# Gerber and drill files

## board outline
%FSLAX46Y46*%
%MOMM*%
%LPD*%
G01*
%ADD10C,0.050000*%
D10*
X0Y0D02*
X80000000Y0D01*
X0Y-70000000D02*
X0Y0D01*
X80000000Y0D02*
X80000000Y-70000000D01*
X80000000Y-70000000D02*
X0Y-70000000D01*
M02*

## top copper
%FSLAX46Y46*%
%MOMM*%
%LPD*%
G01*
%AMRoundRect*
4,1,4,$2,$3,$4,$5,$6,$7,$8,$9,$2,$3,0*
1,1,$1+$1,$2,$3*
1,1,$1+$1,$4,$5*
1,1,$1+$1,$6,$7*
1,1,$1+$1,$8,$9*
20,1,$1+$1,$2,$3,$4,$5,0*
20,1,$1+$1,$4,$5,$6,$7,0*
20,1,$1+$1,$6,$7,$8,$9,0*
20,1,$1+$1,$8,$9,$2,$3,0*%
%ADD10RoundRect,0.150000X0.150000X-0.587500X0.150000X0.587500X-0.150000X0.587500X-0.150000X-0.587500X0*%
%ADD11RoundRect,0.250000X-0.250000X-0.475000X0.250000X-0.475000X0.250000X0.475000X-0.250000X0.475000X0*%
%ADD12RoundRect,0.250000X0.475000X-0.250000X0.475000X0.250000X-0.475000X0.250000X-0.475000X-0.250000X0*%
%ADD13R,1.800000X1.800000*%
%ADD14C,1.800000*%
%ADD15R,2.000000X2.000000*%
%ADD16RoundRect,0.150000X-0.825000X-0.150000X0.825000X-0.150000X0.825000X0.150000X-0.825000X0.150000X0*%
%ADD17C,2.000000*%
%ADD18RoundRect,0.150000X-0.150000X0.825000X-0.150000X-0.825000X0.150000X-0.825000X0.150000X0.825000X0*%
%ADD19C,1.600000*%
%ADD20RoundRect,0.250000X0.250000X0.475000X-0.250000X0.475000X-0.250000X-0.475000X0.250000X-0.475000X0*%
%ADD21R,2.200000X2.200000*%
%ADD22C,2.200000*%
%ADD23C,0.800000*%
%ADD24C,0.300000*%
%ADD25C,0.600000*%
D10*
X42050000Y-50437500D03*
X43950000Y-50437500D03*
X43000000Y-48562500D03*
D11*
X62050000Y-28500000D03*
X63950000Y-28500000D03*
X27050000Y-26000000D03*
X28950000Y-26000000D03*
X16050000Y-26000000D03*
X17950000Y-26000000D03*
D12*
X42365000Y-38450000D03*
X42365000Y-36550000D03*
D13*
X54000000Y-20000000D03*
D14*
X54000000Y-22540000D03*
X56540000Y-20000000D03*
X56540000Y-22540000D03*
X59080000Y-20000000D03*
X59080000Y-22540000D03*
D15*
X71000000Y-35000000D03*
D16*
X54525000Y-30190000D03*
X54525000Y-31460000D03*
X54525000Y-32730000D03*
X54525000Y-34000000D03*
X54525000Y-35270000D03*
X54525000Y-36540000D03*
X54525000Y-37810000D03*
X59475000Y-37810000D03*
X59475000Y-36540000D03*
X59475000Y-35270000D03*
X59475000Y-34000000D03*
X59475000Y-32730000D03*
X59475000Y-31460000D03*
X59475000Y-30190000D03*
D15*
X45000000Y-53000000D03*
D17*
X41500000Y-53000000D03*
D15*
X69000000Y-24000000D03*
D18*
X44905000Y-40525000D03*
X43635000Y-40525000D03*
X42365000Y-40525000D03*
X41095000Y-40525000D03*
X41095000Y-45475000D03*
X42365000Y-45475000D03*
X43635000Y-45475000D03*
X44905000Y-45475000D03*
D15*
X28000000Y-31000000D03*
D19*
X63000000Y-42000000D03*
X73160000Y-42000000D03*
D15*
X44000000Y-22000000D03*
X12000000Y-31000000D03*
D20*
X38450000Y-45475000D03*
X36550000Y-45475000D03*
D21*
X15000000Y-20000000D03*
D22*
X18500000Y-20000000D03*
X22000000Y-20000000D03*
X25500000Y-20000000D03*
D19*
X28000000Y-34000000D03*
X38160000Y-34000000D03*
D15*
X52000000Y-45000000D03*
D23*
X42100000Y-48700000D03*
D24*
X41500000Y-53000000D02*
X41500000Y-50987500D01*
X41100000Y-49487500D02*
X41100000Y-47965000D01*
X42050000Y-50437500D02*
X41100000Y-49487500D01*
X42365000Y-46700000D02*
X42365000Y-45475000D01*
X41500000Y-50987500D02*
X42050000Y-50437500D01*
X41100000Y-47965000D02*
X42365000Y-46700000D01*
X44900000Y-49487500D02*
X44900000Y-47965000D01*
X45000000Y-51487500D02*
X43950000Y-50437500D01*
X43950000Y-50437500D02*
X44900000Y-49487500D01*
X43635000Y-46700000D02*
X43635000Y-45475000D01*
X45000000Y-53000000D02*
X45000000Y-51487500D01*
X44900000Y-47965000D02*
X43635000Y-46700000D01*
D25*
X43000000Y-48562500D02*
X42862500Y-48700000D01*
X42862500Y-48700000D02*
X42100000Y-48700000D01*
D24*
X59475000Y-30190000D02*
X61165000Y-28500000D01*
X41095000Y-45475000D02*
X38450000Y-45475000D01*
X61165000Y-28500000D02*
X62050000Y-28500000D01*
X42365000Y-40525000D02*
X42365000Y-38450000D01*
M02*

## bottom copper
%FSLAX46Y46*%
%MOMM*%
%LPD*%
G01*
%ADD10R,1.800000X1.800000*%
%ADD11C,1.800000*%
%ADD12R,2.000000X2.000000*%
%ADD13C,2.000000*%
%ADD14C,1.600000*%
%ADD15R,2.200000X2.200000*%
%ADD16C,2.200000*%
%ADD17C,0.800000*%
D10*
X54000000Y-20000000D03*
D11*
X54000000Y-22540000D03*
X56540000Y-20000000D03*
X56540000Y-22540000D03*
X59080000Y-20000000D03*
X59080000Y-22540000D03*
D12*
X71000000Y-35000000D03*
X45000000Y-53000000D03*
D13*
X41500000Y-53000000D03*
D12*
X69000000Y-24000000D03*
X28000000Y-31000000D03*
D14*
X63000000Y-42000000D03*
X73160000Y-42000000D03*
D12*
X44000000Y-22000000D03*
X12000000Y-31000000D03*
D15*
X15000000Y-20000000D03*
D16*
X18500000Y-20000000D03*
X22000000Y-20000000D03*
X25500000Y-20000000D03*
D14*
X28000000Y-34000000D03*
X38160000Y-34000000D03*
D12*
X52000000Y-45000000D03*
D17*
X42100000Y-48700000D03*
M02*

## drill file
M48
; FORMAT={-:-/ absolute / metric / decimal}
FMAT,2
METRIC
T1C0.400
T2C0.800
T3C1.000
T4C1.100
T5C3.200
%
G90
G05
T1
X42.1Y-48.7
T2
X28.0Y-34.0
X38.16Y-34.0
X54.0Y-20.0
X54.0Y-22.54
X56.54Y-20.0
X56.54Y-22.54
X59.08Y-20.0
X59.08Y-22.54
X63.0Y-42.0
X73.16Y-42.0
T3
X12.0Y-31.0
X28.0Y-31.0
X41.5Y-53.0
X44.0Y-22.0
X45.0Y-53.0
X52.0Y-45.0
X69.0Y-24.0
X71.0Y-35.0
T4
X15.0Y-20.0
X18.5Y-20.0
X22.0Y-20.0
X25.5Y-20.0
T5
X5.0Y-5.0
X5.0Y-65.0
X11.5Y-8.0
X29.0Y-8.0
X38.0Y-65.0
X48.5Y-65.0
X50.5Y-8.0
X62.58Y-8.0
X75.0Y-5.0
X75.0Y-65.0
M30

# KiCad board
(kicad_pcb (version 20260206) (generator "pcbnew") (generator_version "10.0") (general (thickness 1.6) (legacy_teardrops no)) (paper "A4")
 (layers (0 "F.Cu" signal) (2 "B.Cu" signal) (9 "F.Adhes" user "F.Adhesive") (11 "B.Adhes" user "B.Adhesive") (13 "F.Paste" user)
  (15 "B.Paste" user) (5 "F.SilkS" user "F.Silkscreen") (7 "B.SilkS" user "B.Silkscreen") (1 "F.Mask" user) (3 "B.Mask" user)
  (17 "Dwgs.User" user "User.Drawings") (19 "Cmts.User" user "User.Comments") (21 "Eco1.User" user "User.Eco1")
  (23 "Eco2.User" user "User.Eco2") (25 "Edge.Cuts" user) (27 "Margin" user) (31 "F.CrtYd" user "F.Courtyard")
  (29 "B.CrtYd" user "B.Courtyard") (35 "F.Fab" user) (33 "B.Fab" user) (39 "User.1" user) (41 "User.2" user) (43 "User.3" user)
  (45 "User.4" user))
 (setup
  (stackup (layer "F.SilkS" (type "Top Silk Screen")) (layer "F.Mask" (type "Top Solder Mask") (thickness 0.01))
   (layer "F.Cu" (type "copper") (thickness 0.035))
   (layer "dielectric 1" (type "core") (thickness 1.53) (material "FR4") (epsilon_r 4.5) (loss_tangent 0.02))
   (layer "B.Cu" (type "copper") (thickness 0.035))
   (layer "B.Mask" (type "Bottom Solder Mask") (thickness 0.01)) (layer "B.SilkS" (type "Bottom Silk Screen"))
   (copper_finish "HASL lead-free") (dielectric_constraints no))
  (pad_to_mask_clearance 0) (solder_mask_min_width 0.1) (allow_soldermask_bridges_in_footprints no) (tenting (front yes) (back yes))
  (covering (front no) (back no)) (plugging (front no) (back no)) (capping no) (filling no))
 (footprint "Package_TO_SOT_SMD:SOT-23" (layer "F.Cu") (at 43 49.5 90)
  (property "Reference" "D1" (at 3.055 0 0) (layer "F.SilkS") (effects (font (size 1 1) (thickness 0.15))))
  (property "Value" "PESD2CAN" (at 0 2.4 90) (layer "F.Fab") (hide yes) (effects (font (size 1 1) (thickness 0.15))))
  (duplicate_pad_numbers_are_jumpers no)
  (pad "1" smd roundrect (at -0.9375 -0.95 90) (size 1.475 0.6) (layers "F.Cu" "F.Mask" "F.Paste") (roundrect_rratio 0.25) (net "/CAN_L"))
  (pad "2" smd roundrect (at -0.9375 0.95 90) (size 1.475 0.6) (layers "F.Cu" "F.Mask" "F.Paste") (roundrect_rratio 0.25) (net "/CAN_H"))
  (pad "3" smd roundrect (at 0.9375 0 90) (size 1.475 0.6) (layers "F.Cu" "F.Mask" "F.Paste") (roundrect_rratio 0.25) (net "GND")))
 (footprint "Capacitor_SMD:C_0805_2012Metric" (layer "F.Cu") (at 63 28.5)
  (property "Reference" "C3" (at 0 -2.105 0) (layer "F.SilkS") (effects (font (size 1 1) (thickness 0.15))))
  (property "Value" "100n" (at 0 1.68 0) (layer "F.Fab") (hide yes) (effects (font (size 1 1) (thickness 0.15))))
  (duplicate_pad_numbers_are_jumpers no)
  (pad "1" smd roundrect (at -0.95 0) (size 1 1.45) (layers "F.Cu" "F.Mask" "F.Paste") (roundrect_rratio 0.25) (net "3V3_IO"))
  (pad "2" smd roundrect (at 0.95 0) (size 1 1.45) (layers "F.Cu" "F.Mask" "F.Paste") (roundrect_rratio 0.25) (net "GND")))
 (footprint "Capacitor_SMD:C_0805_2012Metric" (layer "F.Cu") (at 28 26)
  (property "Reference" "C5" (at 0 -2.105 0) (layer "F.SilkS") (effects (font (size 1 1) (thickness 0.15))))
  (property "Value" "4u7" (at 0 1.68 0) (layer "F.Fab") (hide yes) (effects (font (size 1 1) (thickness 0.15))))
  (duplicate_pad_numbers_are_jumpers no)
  (pad "1" smd roundrect (at -0.95 0) (size 1 1.45) (layers "F.Cu" "F.Mask" "F.Paste") (roundrect_rratio 0.25) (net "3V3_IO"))
  (pad "2" smd roundrect (at 0.95 0) (size 1 1.45) (layers "F.Cu" "F.Mask" "F.Paste") (roundrect_rratio 0.25) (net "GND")))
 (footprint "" (layer "F.Cu") (at 75 65)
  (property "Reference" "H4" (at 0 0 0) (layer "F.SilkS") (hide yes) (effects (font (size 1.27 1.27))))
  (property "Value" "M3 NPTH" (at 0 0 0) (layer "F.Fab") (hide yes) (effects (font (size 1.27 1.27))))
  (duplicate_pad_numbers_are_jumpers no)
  (pad "" np_thru_hole circle (at 0 0) (size 3.2 3.2) (drill 3.2) (layers "*.Cu")))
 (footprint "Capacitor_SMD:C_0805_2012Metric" (layer "F.Cu") (at 17 26)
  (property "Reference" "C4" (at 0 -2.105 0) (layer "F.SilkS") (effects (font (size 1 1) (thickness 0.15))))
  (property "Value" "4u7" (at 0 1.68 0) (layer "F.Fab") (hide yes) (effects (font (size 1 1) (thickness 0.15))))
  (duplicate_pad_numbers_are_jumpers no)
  (pad "1" smd roundrect (at -0.95 0) (size 1 1.45) (layers "F.Cu" "F.Mask" "F.Paste") (roundrect_rratio 0.25) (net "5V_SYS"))
  (pad "2" smd roundrect (at 0.95 0) (size 1 1.45) (layers "F.Cu" "F.Mask" "F.Paste") (roundrect_rratio 0.25) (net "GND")))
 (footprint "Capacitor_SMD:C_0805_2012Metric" (layer "F.Cu") (at 42.365 37.5 90)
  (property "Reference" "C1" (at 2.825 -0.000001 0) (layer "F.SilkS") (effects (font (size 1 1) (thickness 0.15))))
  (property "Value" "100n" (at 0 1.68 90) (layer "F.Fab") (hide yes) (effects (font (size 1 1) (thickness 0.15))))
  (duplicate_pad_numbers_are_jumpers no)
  (pad "1" smd roundrect (at -0.95 0 90) (size 1 1.45) (layers "F.Cu" "F.Mask" "F.Paste") (roundrect_rratio 0.25) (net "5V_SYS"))
  (pad "2" smd roundrect (at 0.95 0 90) (size 1 1.45) (layers "F.Cu" "F.Mask" "F.Paste") (roundrect_rratio 0.25) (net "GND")))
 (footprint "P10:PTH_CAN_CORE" (layer "F.Cu") (at 54 20)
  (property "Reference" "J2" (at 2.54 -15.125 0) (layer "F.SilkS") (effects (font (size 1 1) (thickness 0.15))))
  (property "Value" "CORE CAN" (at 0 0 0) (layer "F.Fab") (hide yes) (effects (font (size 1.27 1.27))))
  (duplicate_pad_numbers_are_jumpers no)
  (pad "" np_thru_hole circle (at -3.5 -12) (size 3.2 3.2) (drill 3.2) (layers "*.Cu" "*.Mask"))
  (pad "" np_thru_hole circle (at 8.58 -12) (size 3.2 3.2) (drill 3.2) (layers "*.Cu" "*.Mask"))
  (pad "1" thru_hole rect (at 0 0) (size 1.8 1.8) (drill 0.8) (layers "*.Cu" "*.Mask") (remove_unused_layers no) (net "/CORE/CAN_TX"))
  (pad "2" thru_hole circle (at 0 2.54) (size 1.8 1.8) (drill 0.8) (layers "*.Cu" "*.Mask") (remove_unused_layers no) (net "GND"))
  (pad "3" thru_hole circle (at 2.54 0) (size 1.8 1.8) (drill 0.8) (layers "*.Cu" "*.Mask") (remove_unused_layers no) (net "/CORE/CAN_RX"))
  (pad "4" thru_hole circle (at 2.54 2.54) (size 1.8 1.8) (drill 0.8) (layers "*.Cu" "*.Mask") (remove_unused_layers no)
   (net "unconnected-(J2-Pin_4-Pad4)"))
  (pad "5" thru_hole circle (at 5.08 0) (size 1.8 1.8) (drill 0.8) (layers "*.Cu" "*.Mask") (remove_unused_layers no)
   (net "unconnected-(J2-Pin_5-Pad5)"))
  (pad "6" thru_hole circle (at 5.08 2.54) (size 1.8 1.8) (drill 0.8) (layers "*.Cu" "*.Mask") (remove_unused_layers no)
   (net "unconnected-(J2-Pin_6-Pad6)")))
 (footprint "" (layer "F.Cu") (at 5 65)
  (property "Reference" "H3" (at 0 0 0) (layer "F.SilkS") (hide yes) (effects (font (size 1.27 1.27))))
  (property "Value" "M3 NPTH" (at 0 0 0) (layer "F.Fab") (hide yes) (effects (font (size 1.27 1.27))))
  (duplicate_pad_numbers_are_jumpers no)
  (pad "" np_thru_hole circle (at 0 0) (size 3.2 3.2) (drill 3.2) (layers "*.Cu")))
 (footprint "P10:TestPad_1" (layer "F.Cu") (at 71 35)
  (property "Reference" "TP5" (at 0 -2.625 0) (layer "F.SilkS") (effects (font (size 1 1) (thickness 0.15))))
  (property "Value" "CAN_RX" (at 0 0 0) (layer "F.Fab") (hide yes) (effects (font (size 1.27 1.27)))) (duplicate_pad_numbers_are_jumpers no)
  (pad "1" thru_hole rect (at 0 0) (size 2 2) (drill 1) (layers "*.Cu" "*.Mask") (remove_unused_layers no) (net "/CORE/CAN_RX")))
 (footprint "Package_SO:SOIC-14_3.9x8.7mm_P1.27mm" (layer "F.Cu") (at 57 34)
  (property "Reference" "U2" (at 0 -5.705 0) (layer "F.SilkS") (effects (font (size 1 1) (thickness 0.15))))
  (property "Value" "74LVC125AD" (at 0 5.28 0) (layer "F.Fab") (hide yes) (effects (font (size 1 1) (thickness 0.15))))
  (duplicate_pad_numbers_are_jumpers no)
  (pad "1" smd roundrect (at -2.475 -3.81) (size 1.95 0.6) (layers "F.Cu" "F.Mask" "F.Paste") (roundrect_rratio 0.25) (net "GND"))
  (pad "2" smd roundrect (at -2.475 -2.54) (size 1.95 0.6) (layers "F.Cu" "F.Mask" "F.Paste") (roundrect_rratio 0.25) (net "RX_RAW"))
  (pad "3" smd roundrect (at -2.475 -1.27) (size 1.95 0.6) (layers "F.Cu" "F.Mask" "F.Paste") (roundrect_rratio 0.25) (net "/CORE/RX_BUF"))
  (pad "4" smd roundrect (at -2.475 0) (size 1.95 0.6) (layers "F.Cu" "F.Mask" "F.Paste") (roundrect_rratio 0.25) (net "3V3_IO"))
  (pad "5" smd roundrect (at -2.475 1.27) (size 1.95 0.6) (layers "F.Cu" "F.Mask" "F.Paste") (roundrect_rratio 0.25) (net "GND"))
  (pad "6" smd roundrect (at -2.475 2.54) (size 1.95 0.6) (layers "F.Cu" "F.Mask" "F.Paste") (roundrect_rratio 0.25)
   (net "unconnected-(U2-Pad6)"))
  (pad "7" smd roundrect (at -2.475 3.81) (size 1.95 0.6) (layers "F.Cu" "F.Mask" "F.Paste") (roundrect_rratio 0.25) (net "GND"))
  (pad "8" smd roundrect (at 2.475 3.81) (size 1.95 0.6) (layers "F.Cu" "F.Mask" "F.Paste") (roundrect_rratio 0.25)
   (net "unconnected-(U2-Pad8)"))
  (pad "9" smd roundrect (at 2.475 2.54) (size 1.95 0.6) (layers "F.Cu" "F.Mask" "F.Paste") (roundrect_rratio 0.25) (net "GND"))
  (pad "10" smd roundrect (at 2.475 1.27) (size 1.95 0.6) (layers "F.Cu" "F.Mask" "F.Paste") (roundrect_rratio 0.25) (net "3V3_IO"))
  (pad "11" smd roundrect (at 2.475 0) (size 1.95 0.6) (layers "F.Cu" "F.Mask" "F.Paste") (roundrect_rratio 0.25)
   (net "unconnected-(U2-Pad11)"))
  (pad "12" smd roundrect (at 2.475 -1.27) (size 1.95 0.6) (layers "F.Cu" "F.Mask" "F.Paste") (roundrect_rratio 0.25) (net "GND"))
  (pad "13" smd roundrect (at 2.475 -2.54) (size 1.95 0.6) (layers "F.Cu" "F.Mask" "F.Paste") (roundrect_rratio 0.25) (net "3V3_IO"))
  (pad "14" smd roundrect (at 2.475 -3.81) (size 1.95 0.6) (layers "F.Cu" "F.Mask" "F.Paste") (roundrect_rratio 0.25) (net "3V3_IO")))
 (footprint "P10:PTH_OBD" (layer "F.Cu") (at 45 53 180)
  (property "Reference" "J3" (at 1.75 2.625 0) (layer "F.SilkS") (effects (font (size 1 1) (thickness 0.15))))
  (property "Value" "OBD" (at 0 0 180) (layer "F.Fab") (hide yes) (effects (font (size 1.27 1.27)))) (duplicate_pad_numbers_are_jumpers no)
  (pad "" np_thru_hole circle (at -3.5 -12 180) (size 3.2 3.2) (drill 3.2) (layers "*.Cu" "*.Mask"))
  (pad "" np_thru_hole circle (at 7 -12 180) (size 3.2 3.2) (drill 3.2) (layers "*.Cu" "*.Mask"))
  (pad "1" thru_hole rect (at 0 0 180) (size 2 2) (drill 1) (layers "*.Cu" "*.Mask") (remove_unused_layers no) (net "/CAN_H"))
  (pad "2" thru_hole circle (at 3.5 0 180) (size 2 2) (drill 1) (layers "*.Cu" "*.Mask") (remove_unused_layers no) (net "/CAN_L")))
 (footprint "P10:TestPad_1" (layer "F.Cu") (at 69 24)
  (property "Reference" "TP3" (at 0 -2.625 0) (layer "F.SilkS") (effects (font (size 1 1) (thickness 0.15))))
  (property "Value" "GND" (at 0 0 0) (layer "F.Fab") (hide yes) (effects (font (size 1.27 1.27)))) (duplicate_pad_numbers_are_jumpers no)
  (pad "1" thru_hole rect (at 0 0) (size 2 2) (drill 1) (layers "*.Cu" "*.Mask") (remove_unused_layers no) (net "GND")))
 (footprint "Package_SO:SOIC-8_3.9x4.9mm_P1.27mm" (layer "F.Cu") (at 43 43 -90)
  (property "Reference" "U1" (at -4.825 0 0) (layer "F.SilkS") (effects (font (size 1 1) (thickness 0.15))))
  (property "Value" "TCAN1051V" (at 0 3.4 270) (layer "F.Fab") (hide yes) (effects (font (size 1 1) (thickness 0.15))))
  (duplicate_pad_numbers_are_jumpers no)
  (pad "1" smd roundrect (at -2.475 -1.905 270) (size 1.95 0.6) (layers "F.Cu" "F.Mask" "F.Paste") (roundrect_rratio 0.25) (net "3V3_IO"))
  (pad "2" smd roundrect (at -2.475 -0.635 270) (size 1.95 0.6) (layers "F.Cu" "F.Mask" "F.Paste") (roundrect_rratio 0.25) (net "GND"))
  (pad "3" smd roundrect (at -2.475 0.635 270) (size 1.95 0.6) (layers "F.Cu" "F.Mask" "F.Paste") (roundrect_rratio 0.25) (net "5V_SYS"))
  (pad "4" smd roundrect (at -2.475 1.905 270) (size 1.95 0.6) (layers "F.Cu" "F.Mask" "F.Paste") (roundrect_rratio 0.25) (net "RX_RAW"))
  (pad "5" smd roundrect (at 2.475 1.905 270) (size 1.95 0.6) (layers "F.Cu" "F.Mask" "F.Paste") (roundrect_rratio 0.25) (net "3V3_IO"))
  (pad "6" smd roundrect (at 2.475 0.635 270) (size 1.95 0.6) (layers "F.Cu" "F.Mask" "F.Paste") (roundrect_rratio 0.25) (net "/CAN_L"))
  (pad "7" smd roundrect (at 2.475 -0.635 270) (size 1.95 0.6) (layers "F.Cu" "F.Mask" "F.Paste") (roundrect_rratio 0.25) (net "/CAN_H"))
  (pad "8" smd roundrect (at 2.475 -1.905 270) (size 1.95 0.6) (layers "F.Cu" "F.Mask" "F.Paste") (roundrect_rratio 0.25) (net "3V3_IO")))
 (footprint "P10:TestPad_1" (layer "F.Cu") (at 28 31)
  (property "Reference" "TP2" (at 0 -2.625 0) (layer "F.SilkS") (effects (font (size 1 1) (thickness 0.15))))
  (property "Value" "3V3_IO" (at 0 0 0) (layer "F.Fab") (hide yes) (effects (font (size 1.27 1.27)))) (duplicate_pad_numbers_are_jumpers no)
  (pad "1" thru_hole rect (at 0 0) (size 2 2) (drill 1) (layers "*.Cu" "*.Mask") (remove_unused_layers no) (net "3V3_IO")))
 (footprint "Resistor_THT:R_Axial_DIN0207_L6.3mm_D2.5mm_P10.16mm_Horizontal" (layer "F.Cu") (at 63 42)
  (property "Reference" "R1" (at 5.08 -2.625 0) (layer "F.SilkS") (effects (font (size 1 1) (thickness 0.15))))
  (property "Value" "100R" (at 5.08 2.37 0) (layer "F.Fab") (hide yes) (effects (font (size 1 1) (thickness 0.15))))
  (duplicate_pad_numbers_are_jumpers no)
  (pad "1" thru_hole circle (at 0 0) (size 1.6 1.6) (drill 0.8) (layers "*.Cu" "*.Mask") (remove_unused_layers no) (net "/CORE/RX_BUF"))
  (pad "2" thru_hole circle (at 10.16 0) (size 1.6 1.6) (drill 0.8) (layers "*.Cu" "*.Mask") (remove_unused_layers no) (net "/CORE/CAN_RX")))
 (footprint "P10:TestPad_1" (layer "F.Cu") (at 44 22)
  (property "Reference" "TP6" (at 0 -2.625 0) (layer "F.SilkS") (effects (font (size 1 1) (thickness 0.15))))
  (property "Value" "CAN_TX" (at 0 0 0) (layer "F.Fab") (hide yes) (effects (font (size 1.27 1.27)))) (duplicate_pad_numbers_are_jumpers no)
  (pad "1" thru_hole rect (at 0 0) (size 2 2) (drill 1) (layers "*.Cu" "*.Mask") (remove_unused_layers no) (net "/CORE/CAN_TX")))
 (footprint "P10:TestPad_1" (layer "F.Cu") (at 12 31)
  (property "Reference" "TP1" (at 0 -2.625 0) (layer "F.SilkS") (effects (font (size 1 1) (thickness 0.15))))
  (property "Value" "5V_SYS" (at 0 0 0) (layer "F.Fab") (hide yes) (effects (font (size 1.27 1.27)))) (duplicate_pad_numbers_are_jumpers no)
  (pad "1" thru_hole rect (at 0 0) (size 2 2) (drill 1) (layers "*.Cu" "*.Mask") (remove_unused_layers no) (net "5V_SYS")))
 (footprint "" (layer "F.Cu") (at 5 5)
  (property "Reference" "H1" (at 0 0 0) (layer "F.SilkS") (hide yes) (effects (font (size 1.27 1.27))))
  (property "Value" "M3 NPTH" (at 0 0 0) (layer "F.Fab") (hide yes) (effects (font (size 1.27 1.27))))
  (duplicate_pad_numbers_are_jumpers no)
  (pad "" np_thru_hole circle (at 0 0) (size 3.2 3.2) (drill 3.2) (layers "*.Cu")))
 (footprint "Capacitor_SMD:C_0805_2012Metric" (layer "F.Cu") (at 37.5 45.475 180)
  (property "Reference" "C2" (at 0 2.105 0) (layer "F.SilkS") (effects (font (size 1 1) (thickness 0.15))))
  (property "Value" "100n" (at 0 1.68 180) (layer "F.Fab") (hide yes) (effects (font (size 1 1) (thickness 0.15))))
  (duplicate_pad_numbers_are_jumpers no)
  (pad "1" smd roundrect (at -0.95 0 180) (size 1 1.45) (layers "F.Cu" "F.Mask" "F.Paste") (roundrect_rratio 0.25) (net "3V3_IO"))
  (pad "2" smd roundrect (at 0.95 0 180) (size 1 1.45) (layers "F.Cu" "F.Mask" "F.Paste") (roundrect_rratio 0.25) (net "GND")))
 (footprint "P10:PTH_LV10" (layer "F.Cu") (at 15 20)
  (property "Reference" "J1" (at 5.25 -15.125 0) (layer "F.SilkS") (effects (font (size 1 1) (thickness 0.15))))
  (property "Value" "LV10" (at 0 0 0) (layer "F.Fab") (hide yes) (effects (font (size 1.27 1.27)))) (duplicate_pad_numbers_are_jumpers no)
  (pad "" np_thru_hole circle (at -3.5 -12) (size 3.2 3.2) (drill 3.2) (layers "*.Cu" "*.Mask"))
  (pad "" np_thru_hole circle (at 14 -12) (size 3.2 3.2) (drill 3.2) (layers "*.Cu" "*.Mask"))
  (pad "1" thru_hole rect (at 0 0) (size 2.2 2.2) (drill 1.1) (layers "*.Cu" "*.Mask") (remove_unused_layers no) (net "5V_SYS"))
  (pad "2" thru_hole circle (at 3.5 0) (size 2.2 2.2) (drill 1.1) (layers "*.Cu" "*.Mask") (remove_unused_layers no) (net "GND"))
  (pad "3" thru_hole circle (at 7 0) (size 2.2 2.2) (drill 1.1) (layers "*.Cu" "*.Mask") (remove_unused_layers no) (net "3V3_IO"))
  (pad "4" thru_hole circle (at 10.5 0) (size 2.2 2.2) (drill 1.1) (layers "*.Cu" "*.Mask") (remove_unused_layers no) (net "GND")))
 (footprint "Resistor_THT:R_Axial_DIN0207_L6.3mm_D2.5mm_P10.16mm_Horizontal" (layer "F.Cu") (at 28 34)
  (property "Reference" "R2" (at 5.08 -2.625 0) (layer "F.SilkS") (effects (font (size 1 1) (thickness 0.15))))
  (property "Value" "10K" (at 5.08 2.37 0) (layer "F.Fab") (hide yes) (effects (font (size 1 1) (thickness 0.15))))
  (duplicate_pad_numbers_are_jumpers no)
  (pad "1" thru_hole circle (at 0 0) (size 1.6 1.6) (drill 0.8) (layers "*.Cu" "*.Mask") (remove_unused_layers no) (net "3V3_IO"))
  (pad "2" thru_hole circle (at 10.16 0) (size 1.6 1.6) (drill 0.8) (layers "*.Cu" "*.Mask") (remove_unused_layers no) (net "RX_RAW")))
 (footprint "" (layer "F.Cu") (at 75 5)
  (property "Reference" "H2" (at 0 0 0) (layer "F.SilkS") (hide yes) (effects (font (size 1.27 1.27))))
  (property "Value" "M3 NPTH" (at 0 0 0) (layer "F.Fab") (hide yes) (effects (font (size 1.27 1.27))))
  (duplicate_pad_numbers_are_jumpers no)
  (pad "" np_thru_hole circle (at 0 0) (size 3.2 3.2) (drill 3.2) (layers "*.Cu")))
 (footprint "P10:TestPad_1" (layer "F.Cu") (at 52 45)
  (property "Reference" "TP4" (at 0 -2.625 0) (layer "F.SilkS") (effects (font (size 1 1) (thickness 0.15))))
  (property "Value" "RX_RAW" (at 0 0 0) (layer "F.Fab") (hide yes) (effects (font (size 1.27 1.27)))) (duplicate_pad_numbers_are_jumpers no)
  (pad "1" thru_hole rect (at 0 0) (size 2 2) (drill 1) (layers "*.Cu" "*.Mask") (remove_unused_layers no) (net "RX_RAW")))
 (gr_line (start 0 0) (end 80 0) (stroke (width 0.05) (type default)) (layer "Edge.Cuts"))
 (gr_line (start 0 70) (end 0 0) (stroke (width 0.05) (type default)) (layer "Edge.Cuts"))
 (gr_line (start 80 0) (end 80 70) (stroke (width 0.05) (type default)) (layer "Edge.Cuts"))
 (gr_line (start 80 70) (end 0 70) (stroke (width 0.05) (type default)) (layer "Edge.Cuts"))
 (segment (start 41.5 53) (end 41.5 50.9875) (width 0.3) (locked yes) (layer "F.Cu") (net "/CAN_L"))
 (segment (start 41.1 49.4875) (end 41.1 47.965) (width 0.3) (locked yes) (layer "F.Cu") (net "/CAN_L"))
 (segment (start 42.05 50.4375) (end 41.1 49.4875) (width 0.3) (locked yes) (layer "F.Cu") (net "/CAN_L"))
 (segment (start 42.365 46.7) (end 42.365 45.475) (width 0.3) (locked yes) (layer "F.Cu") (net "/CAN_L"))
 (segment (start 41.5 50.9875) (end 42.05 50.4375) (width 0.3) (locked yes) (layer "F.Cu") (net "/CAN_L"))
 (segment (start 41.1 47.965) (end 42.365 46.7) (width 0.3) (locked yes) (layer "F.Cu") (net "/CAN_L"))
 (segment (start 44.9 49.4875) (end 44.9 47.965) (width 0.3) (locked yes) (layer "F.Cu") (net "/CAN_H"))
 (segment (start 45 51.4875) (end 43.95 50.4375) (width 0.3) (locked yes) (layer "F.Cu") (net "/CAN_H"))
 (segment (start 43.95 50.4375) (end 44.9 49.4875) (width 0.3) (locked yes) (layer "F.Cu") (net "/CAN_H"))
 (segment (start 43.635 46.7) (end 43.635 45.475) (width 0.3) (locked yes) (layer "F.Cu") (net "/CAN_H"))
 (segment (start 45 53) (end 45 51.4875) (width 0.3) (locked yes) (layer "F.Cu") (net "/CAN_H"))
 (segment (start 44.9 47.965) (end 43.635 46.7) (width 0.3) (locked yes) (layer "F.Cu") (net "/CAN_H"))
 (segment (start 43 48.5625) (end 42.8625 48.7) (width 0.6) (locked yes) (layer "F.Cu") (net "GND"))
 (segment (start 42.8625 48.7) (end 42.1 48.7) (width 0.6) (locked yes) (layer "F.Cu") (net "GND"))
 (via (at 42.1 48.7) (size 0.8) (drill 0.4) (layers "F.Cu" "B.Cu") (locked yes) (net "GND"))
 (segment (start 59.475 30.19) (end 61.165 28.5) (width 0.3) (locked yes) (layer "F.Cu") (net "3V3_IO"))
 (segment (start 41.095 45.475) (end 38.45 45.475) (width 0.3) (locked yes) (layer "F.Cu") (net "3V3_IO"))
 (segment (start 61.165 28.5) (end 62.05 28.5) (width 0.3) (locked yes) (layer "F.Cu") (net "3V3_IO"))
 (segment (start 42.365 40.525) (end 42.365 38.45) (width 0.3) (locked yes) (layer "F.Cu") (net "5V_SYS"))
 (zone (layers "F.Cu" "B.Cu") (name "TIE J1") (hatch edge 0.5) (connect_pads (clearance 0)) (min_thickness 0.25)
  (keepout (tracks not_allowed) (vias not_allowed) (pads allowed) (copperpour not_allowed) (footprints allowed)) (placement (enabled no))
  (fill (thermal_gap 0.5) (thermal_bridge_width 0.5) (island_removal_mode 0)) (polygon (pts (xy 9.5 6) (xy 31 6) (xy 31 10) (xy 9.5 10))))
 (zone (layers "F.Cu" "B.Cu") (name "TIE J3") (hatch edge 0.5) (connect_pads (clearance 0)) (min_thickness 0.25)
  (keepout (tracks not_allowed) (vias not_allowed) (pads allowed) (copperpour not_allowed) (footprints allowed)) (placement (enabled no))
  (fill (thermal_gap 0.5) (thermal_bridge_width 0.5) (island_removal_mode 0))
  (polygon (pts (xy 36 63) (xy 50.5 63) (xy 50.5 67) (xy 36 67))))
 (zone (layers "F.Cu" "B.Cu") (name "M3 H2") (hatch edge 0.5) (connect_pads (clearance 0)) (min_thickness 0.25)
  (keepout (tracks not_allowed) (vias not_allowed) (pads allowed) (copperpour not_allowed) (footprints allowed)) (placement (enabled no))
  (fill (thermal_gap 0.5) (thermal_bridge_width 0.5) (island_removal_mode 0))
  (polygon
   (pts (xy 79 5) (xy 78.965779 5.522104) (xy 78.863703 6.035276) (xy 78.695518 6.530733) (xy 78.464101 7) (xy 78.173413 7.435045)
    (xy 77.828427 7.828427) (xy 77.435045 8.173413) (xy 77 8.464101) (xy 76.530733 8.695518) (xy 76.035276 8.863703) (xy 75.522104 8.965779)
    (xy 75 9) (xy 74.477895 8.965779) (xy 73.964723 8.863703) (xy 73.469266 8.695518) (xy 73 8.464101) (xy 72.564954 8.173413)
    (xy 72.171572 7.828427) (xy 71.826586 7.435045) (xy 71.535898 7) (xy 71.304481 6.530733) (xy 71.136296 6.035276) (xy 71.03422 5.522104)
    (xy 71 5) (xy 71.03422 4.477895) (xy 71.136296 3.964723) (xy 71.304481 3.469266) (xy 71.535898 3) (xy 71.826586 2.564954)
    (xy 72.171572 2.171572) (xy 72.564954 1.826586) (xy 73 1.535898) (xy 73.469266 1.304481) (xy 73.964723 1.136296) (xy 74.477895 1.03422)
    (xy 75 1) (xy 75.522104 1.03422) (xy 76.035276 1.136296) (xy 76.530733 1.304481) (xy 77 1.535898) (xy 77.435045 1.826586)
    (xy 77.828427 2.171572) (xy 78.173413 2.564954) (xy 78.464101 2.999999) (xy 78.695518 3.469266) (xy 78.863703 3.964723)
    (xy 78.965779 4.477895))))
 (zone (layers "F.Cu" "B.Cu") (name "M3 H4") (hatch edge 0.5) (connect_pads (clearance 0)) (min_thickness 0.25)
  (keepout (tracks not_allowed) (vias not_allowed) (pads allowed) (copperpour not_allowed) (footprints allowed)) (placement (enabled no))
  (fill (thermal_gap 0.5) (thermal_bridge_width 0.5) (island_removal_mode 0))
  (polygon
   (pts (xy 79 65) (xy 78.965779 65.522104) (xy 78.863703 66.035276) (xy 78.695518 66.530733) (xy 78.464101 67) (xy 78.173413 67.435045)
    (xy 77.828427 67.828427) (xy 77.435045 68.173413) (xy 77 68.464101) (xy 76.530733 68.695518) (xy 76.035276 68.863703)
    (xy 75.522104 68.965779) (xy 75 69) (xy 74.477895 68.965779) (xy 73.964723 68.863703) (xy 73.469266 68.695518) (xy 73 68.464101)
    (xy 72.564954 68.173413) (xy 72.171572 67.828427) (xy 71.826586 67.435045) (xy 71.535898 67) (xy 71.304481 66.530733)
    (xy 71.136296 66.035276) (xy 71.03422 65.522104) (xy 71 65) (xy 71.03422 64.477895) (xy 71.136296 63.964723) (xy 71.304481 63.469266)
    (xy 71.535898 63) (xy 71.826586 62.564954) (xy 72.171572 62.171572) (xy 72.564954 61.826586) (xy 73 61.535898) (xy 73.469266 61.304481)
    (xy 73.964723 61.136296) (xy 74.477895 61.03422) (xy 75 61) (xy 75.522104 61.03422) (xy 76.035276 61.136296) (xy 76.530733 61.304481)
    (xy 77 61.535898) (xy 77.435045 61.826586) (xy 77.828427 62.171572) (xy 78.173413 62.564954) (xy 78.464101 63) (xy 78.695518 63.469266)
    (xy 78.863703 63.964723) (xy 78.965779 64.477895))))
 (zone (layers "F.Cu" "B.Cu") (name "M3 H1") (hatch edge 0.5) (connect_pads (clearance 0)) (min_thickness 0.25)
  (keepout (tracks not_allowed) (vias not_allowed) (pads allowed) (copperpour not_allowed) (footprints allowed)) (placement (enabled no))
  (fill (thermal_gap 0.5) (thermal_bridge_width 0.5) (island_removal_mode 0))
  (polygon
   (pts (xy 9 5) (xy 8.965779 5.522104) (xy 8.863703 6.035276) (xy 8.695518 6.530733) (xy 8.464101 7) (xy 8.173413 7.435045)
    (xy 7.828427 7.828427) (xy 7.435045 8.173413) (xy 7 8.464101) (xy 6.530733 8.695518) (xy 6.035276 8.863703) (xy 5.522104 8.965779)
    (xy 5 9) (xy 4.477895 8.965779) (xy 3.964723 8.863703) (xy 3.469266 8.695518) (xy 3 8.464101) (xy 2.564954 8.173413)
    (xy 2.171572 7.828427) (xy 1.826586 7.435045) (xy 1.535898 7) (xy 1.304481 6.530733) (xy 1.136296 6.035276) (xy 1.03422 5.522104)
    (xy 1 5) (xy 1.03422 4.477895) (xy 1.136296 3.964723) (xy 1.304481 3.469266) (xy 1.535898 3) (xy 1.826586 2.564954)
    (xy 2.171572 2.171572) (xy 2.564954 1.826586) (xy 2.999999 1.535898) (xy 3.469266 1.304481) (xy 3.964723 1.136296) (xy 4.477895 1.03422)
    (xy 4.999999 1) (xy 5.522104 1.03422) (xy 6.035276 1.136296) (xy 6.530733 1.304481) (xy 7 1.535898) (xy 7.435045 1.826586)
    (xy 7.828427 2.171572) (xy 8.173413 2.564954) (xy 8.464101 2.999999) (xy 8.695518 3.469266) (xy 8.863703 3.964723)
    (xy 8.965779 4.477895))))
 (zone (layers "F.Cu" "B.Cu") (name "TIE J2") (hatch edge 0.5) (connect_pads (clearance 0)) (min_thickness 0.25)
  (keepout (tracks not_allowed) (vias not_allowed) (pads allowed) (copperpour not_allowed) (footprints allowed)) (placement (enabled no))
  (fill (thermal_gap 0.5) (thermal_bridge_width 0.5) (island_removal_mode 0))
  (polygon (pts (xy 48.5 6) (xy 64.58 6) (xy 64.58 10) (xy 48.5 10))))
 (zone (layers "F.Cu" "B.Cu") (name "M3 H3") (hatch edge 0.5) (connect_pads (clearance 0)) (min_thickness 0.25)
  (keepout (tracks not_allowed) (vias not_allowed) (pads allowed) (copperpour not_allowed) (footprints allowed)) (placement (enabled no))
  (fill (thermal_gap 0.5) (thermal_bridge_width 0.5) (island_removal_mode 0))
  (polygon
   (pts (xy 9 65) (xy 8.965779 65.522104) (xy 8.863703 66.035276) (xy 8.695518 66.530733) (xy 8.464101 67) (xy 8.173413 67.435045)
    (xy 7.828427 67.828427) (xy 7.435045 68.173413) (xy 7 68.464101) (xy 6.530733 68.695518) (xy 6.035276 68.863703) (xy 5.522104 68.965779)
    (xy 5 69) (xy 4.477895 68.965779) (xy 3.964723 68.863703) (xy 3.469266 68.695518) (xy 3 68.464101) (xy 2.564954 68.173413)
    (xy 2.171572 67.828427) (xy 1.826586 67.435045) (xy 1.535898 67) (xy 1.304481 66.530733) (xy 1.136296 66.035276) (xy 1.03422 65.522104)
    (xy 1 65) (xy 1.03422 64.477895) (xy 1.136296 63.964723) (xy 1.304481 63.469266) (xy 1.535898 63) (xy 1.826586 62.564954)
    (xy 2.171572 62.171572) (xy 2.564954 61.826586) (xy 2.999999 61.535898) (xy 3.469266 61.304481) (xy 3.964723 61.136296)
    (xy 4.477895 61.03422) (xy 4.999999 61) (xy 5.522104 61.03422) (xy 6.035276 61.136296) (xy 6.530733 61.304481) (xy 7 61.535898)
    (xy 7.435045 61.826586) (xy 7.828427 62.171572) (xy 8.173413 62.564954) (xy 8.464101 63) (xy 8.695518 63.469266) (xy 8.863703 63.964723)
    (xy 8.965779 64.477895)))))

